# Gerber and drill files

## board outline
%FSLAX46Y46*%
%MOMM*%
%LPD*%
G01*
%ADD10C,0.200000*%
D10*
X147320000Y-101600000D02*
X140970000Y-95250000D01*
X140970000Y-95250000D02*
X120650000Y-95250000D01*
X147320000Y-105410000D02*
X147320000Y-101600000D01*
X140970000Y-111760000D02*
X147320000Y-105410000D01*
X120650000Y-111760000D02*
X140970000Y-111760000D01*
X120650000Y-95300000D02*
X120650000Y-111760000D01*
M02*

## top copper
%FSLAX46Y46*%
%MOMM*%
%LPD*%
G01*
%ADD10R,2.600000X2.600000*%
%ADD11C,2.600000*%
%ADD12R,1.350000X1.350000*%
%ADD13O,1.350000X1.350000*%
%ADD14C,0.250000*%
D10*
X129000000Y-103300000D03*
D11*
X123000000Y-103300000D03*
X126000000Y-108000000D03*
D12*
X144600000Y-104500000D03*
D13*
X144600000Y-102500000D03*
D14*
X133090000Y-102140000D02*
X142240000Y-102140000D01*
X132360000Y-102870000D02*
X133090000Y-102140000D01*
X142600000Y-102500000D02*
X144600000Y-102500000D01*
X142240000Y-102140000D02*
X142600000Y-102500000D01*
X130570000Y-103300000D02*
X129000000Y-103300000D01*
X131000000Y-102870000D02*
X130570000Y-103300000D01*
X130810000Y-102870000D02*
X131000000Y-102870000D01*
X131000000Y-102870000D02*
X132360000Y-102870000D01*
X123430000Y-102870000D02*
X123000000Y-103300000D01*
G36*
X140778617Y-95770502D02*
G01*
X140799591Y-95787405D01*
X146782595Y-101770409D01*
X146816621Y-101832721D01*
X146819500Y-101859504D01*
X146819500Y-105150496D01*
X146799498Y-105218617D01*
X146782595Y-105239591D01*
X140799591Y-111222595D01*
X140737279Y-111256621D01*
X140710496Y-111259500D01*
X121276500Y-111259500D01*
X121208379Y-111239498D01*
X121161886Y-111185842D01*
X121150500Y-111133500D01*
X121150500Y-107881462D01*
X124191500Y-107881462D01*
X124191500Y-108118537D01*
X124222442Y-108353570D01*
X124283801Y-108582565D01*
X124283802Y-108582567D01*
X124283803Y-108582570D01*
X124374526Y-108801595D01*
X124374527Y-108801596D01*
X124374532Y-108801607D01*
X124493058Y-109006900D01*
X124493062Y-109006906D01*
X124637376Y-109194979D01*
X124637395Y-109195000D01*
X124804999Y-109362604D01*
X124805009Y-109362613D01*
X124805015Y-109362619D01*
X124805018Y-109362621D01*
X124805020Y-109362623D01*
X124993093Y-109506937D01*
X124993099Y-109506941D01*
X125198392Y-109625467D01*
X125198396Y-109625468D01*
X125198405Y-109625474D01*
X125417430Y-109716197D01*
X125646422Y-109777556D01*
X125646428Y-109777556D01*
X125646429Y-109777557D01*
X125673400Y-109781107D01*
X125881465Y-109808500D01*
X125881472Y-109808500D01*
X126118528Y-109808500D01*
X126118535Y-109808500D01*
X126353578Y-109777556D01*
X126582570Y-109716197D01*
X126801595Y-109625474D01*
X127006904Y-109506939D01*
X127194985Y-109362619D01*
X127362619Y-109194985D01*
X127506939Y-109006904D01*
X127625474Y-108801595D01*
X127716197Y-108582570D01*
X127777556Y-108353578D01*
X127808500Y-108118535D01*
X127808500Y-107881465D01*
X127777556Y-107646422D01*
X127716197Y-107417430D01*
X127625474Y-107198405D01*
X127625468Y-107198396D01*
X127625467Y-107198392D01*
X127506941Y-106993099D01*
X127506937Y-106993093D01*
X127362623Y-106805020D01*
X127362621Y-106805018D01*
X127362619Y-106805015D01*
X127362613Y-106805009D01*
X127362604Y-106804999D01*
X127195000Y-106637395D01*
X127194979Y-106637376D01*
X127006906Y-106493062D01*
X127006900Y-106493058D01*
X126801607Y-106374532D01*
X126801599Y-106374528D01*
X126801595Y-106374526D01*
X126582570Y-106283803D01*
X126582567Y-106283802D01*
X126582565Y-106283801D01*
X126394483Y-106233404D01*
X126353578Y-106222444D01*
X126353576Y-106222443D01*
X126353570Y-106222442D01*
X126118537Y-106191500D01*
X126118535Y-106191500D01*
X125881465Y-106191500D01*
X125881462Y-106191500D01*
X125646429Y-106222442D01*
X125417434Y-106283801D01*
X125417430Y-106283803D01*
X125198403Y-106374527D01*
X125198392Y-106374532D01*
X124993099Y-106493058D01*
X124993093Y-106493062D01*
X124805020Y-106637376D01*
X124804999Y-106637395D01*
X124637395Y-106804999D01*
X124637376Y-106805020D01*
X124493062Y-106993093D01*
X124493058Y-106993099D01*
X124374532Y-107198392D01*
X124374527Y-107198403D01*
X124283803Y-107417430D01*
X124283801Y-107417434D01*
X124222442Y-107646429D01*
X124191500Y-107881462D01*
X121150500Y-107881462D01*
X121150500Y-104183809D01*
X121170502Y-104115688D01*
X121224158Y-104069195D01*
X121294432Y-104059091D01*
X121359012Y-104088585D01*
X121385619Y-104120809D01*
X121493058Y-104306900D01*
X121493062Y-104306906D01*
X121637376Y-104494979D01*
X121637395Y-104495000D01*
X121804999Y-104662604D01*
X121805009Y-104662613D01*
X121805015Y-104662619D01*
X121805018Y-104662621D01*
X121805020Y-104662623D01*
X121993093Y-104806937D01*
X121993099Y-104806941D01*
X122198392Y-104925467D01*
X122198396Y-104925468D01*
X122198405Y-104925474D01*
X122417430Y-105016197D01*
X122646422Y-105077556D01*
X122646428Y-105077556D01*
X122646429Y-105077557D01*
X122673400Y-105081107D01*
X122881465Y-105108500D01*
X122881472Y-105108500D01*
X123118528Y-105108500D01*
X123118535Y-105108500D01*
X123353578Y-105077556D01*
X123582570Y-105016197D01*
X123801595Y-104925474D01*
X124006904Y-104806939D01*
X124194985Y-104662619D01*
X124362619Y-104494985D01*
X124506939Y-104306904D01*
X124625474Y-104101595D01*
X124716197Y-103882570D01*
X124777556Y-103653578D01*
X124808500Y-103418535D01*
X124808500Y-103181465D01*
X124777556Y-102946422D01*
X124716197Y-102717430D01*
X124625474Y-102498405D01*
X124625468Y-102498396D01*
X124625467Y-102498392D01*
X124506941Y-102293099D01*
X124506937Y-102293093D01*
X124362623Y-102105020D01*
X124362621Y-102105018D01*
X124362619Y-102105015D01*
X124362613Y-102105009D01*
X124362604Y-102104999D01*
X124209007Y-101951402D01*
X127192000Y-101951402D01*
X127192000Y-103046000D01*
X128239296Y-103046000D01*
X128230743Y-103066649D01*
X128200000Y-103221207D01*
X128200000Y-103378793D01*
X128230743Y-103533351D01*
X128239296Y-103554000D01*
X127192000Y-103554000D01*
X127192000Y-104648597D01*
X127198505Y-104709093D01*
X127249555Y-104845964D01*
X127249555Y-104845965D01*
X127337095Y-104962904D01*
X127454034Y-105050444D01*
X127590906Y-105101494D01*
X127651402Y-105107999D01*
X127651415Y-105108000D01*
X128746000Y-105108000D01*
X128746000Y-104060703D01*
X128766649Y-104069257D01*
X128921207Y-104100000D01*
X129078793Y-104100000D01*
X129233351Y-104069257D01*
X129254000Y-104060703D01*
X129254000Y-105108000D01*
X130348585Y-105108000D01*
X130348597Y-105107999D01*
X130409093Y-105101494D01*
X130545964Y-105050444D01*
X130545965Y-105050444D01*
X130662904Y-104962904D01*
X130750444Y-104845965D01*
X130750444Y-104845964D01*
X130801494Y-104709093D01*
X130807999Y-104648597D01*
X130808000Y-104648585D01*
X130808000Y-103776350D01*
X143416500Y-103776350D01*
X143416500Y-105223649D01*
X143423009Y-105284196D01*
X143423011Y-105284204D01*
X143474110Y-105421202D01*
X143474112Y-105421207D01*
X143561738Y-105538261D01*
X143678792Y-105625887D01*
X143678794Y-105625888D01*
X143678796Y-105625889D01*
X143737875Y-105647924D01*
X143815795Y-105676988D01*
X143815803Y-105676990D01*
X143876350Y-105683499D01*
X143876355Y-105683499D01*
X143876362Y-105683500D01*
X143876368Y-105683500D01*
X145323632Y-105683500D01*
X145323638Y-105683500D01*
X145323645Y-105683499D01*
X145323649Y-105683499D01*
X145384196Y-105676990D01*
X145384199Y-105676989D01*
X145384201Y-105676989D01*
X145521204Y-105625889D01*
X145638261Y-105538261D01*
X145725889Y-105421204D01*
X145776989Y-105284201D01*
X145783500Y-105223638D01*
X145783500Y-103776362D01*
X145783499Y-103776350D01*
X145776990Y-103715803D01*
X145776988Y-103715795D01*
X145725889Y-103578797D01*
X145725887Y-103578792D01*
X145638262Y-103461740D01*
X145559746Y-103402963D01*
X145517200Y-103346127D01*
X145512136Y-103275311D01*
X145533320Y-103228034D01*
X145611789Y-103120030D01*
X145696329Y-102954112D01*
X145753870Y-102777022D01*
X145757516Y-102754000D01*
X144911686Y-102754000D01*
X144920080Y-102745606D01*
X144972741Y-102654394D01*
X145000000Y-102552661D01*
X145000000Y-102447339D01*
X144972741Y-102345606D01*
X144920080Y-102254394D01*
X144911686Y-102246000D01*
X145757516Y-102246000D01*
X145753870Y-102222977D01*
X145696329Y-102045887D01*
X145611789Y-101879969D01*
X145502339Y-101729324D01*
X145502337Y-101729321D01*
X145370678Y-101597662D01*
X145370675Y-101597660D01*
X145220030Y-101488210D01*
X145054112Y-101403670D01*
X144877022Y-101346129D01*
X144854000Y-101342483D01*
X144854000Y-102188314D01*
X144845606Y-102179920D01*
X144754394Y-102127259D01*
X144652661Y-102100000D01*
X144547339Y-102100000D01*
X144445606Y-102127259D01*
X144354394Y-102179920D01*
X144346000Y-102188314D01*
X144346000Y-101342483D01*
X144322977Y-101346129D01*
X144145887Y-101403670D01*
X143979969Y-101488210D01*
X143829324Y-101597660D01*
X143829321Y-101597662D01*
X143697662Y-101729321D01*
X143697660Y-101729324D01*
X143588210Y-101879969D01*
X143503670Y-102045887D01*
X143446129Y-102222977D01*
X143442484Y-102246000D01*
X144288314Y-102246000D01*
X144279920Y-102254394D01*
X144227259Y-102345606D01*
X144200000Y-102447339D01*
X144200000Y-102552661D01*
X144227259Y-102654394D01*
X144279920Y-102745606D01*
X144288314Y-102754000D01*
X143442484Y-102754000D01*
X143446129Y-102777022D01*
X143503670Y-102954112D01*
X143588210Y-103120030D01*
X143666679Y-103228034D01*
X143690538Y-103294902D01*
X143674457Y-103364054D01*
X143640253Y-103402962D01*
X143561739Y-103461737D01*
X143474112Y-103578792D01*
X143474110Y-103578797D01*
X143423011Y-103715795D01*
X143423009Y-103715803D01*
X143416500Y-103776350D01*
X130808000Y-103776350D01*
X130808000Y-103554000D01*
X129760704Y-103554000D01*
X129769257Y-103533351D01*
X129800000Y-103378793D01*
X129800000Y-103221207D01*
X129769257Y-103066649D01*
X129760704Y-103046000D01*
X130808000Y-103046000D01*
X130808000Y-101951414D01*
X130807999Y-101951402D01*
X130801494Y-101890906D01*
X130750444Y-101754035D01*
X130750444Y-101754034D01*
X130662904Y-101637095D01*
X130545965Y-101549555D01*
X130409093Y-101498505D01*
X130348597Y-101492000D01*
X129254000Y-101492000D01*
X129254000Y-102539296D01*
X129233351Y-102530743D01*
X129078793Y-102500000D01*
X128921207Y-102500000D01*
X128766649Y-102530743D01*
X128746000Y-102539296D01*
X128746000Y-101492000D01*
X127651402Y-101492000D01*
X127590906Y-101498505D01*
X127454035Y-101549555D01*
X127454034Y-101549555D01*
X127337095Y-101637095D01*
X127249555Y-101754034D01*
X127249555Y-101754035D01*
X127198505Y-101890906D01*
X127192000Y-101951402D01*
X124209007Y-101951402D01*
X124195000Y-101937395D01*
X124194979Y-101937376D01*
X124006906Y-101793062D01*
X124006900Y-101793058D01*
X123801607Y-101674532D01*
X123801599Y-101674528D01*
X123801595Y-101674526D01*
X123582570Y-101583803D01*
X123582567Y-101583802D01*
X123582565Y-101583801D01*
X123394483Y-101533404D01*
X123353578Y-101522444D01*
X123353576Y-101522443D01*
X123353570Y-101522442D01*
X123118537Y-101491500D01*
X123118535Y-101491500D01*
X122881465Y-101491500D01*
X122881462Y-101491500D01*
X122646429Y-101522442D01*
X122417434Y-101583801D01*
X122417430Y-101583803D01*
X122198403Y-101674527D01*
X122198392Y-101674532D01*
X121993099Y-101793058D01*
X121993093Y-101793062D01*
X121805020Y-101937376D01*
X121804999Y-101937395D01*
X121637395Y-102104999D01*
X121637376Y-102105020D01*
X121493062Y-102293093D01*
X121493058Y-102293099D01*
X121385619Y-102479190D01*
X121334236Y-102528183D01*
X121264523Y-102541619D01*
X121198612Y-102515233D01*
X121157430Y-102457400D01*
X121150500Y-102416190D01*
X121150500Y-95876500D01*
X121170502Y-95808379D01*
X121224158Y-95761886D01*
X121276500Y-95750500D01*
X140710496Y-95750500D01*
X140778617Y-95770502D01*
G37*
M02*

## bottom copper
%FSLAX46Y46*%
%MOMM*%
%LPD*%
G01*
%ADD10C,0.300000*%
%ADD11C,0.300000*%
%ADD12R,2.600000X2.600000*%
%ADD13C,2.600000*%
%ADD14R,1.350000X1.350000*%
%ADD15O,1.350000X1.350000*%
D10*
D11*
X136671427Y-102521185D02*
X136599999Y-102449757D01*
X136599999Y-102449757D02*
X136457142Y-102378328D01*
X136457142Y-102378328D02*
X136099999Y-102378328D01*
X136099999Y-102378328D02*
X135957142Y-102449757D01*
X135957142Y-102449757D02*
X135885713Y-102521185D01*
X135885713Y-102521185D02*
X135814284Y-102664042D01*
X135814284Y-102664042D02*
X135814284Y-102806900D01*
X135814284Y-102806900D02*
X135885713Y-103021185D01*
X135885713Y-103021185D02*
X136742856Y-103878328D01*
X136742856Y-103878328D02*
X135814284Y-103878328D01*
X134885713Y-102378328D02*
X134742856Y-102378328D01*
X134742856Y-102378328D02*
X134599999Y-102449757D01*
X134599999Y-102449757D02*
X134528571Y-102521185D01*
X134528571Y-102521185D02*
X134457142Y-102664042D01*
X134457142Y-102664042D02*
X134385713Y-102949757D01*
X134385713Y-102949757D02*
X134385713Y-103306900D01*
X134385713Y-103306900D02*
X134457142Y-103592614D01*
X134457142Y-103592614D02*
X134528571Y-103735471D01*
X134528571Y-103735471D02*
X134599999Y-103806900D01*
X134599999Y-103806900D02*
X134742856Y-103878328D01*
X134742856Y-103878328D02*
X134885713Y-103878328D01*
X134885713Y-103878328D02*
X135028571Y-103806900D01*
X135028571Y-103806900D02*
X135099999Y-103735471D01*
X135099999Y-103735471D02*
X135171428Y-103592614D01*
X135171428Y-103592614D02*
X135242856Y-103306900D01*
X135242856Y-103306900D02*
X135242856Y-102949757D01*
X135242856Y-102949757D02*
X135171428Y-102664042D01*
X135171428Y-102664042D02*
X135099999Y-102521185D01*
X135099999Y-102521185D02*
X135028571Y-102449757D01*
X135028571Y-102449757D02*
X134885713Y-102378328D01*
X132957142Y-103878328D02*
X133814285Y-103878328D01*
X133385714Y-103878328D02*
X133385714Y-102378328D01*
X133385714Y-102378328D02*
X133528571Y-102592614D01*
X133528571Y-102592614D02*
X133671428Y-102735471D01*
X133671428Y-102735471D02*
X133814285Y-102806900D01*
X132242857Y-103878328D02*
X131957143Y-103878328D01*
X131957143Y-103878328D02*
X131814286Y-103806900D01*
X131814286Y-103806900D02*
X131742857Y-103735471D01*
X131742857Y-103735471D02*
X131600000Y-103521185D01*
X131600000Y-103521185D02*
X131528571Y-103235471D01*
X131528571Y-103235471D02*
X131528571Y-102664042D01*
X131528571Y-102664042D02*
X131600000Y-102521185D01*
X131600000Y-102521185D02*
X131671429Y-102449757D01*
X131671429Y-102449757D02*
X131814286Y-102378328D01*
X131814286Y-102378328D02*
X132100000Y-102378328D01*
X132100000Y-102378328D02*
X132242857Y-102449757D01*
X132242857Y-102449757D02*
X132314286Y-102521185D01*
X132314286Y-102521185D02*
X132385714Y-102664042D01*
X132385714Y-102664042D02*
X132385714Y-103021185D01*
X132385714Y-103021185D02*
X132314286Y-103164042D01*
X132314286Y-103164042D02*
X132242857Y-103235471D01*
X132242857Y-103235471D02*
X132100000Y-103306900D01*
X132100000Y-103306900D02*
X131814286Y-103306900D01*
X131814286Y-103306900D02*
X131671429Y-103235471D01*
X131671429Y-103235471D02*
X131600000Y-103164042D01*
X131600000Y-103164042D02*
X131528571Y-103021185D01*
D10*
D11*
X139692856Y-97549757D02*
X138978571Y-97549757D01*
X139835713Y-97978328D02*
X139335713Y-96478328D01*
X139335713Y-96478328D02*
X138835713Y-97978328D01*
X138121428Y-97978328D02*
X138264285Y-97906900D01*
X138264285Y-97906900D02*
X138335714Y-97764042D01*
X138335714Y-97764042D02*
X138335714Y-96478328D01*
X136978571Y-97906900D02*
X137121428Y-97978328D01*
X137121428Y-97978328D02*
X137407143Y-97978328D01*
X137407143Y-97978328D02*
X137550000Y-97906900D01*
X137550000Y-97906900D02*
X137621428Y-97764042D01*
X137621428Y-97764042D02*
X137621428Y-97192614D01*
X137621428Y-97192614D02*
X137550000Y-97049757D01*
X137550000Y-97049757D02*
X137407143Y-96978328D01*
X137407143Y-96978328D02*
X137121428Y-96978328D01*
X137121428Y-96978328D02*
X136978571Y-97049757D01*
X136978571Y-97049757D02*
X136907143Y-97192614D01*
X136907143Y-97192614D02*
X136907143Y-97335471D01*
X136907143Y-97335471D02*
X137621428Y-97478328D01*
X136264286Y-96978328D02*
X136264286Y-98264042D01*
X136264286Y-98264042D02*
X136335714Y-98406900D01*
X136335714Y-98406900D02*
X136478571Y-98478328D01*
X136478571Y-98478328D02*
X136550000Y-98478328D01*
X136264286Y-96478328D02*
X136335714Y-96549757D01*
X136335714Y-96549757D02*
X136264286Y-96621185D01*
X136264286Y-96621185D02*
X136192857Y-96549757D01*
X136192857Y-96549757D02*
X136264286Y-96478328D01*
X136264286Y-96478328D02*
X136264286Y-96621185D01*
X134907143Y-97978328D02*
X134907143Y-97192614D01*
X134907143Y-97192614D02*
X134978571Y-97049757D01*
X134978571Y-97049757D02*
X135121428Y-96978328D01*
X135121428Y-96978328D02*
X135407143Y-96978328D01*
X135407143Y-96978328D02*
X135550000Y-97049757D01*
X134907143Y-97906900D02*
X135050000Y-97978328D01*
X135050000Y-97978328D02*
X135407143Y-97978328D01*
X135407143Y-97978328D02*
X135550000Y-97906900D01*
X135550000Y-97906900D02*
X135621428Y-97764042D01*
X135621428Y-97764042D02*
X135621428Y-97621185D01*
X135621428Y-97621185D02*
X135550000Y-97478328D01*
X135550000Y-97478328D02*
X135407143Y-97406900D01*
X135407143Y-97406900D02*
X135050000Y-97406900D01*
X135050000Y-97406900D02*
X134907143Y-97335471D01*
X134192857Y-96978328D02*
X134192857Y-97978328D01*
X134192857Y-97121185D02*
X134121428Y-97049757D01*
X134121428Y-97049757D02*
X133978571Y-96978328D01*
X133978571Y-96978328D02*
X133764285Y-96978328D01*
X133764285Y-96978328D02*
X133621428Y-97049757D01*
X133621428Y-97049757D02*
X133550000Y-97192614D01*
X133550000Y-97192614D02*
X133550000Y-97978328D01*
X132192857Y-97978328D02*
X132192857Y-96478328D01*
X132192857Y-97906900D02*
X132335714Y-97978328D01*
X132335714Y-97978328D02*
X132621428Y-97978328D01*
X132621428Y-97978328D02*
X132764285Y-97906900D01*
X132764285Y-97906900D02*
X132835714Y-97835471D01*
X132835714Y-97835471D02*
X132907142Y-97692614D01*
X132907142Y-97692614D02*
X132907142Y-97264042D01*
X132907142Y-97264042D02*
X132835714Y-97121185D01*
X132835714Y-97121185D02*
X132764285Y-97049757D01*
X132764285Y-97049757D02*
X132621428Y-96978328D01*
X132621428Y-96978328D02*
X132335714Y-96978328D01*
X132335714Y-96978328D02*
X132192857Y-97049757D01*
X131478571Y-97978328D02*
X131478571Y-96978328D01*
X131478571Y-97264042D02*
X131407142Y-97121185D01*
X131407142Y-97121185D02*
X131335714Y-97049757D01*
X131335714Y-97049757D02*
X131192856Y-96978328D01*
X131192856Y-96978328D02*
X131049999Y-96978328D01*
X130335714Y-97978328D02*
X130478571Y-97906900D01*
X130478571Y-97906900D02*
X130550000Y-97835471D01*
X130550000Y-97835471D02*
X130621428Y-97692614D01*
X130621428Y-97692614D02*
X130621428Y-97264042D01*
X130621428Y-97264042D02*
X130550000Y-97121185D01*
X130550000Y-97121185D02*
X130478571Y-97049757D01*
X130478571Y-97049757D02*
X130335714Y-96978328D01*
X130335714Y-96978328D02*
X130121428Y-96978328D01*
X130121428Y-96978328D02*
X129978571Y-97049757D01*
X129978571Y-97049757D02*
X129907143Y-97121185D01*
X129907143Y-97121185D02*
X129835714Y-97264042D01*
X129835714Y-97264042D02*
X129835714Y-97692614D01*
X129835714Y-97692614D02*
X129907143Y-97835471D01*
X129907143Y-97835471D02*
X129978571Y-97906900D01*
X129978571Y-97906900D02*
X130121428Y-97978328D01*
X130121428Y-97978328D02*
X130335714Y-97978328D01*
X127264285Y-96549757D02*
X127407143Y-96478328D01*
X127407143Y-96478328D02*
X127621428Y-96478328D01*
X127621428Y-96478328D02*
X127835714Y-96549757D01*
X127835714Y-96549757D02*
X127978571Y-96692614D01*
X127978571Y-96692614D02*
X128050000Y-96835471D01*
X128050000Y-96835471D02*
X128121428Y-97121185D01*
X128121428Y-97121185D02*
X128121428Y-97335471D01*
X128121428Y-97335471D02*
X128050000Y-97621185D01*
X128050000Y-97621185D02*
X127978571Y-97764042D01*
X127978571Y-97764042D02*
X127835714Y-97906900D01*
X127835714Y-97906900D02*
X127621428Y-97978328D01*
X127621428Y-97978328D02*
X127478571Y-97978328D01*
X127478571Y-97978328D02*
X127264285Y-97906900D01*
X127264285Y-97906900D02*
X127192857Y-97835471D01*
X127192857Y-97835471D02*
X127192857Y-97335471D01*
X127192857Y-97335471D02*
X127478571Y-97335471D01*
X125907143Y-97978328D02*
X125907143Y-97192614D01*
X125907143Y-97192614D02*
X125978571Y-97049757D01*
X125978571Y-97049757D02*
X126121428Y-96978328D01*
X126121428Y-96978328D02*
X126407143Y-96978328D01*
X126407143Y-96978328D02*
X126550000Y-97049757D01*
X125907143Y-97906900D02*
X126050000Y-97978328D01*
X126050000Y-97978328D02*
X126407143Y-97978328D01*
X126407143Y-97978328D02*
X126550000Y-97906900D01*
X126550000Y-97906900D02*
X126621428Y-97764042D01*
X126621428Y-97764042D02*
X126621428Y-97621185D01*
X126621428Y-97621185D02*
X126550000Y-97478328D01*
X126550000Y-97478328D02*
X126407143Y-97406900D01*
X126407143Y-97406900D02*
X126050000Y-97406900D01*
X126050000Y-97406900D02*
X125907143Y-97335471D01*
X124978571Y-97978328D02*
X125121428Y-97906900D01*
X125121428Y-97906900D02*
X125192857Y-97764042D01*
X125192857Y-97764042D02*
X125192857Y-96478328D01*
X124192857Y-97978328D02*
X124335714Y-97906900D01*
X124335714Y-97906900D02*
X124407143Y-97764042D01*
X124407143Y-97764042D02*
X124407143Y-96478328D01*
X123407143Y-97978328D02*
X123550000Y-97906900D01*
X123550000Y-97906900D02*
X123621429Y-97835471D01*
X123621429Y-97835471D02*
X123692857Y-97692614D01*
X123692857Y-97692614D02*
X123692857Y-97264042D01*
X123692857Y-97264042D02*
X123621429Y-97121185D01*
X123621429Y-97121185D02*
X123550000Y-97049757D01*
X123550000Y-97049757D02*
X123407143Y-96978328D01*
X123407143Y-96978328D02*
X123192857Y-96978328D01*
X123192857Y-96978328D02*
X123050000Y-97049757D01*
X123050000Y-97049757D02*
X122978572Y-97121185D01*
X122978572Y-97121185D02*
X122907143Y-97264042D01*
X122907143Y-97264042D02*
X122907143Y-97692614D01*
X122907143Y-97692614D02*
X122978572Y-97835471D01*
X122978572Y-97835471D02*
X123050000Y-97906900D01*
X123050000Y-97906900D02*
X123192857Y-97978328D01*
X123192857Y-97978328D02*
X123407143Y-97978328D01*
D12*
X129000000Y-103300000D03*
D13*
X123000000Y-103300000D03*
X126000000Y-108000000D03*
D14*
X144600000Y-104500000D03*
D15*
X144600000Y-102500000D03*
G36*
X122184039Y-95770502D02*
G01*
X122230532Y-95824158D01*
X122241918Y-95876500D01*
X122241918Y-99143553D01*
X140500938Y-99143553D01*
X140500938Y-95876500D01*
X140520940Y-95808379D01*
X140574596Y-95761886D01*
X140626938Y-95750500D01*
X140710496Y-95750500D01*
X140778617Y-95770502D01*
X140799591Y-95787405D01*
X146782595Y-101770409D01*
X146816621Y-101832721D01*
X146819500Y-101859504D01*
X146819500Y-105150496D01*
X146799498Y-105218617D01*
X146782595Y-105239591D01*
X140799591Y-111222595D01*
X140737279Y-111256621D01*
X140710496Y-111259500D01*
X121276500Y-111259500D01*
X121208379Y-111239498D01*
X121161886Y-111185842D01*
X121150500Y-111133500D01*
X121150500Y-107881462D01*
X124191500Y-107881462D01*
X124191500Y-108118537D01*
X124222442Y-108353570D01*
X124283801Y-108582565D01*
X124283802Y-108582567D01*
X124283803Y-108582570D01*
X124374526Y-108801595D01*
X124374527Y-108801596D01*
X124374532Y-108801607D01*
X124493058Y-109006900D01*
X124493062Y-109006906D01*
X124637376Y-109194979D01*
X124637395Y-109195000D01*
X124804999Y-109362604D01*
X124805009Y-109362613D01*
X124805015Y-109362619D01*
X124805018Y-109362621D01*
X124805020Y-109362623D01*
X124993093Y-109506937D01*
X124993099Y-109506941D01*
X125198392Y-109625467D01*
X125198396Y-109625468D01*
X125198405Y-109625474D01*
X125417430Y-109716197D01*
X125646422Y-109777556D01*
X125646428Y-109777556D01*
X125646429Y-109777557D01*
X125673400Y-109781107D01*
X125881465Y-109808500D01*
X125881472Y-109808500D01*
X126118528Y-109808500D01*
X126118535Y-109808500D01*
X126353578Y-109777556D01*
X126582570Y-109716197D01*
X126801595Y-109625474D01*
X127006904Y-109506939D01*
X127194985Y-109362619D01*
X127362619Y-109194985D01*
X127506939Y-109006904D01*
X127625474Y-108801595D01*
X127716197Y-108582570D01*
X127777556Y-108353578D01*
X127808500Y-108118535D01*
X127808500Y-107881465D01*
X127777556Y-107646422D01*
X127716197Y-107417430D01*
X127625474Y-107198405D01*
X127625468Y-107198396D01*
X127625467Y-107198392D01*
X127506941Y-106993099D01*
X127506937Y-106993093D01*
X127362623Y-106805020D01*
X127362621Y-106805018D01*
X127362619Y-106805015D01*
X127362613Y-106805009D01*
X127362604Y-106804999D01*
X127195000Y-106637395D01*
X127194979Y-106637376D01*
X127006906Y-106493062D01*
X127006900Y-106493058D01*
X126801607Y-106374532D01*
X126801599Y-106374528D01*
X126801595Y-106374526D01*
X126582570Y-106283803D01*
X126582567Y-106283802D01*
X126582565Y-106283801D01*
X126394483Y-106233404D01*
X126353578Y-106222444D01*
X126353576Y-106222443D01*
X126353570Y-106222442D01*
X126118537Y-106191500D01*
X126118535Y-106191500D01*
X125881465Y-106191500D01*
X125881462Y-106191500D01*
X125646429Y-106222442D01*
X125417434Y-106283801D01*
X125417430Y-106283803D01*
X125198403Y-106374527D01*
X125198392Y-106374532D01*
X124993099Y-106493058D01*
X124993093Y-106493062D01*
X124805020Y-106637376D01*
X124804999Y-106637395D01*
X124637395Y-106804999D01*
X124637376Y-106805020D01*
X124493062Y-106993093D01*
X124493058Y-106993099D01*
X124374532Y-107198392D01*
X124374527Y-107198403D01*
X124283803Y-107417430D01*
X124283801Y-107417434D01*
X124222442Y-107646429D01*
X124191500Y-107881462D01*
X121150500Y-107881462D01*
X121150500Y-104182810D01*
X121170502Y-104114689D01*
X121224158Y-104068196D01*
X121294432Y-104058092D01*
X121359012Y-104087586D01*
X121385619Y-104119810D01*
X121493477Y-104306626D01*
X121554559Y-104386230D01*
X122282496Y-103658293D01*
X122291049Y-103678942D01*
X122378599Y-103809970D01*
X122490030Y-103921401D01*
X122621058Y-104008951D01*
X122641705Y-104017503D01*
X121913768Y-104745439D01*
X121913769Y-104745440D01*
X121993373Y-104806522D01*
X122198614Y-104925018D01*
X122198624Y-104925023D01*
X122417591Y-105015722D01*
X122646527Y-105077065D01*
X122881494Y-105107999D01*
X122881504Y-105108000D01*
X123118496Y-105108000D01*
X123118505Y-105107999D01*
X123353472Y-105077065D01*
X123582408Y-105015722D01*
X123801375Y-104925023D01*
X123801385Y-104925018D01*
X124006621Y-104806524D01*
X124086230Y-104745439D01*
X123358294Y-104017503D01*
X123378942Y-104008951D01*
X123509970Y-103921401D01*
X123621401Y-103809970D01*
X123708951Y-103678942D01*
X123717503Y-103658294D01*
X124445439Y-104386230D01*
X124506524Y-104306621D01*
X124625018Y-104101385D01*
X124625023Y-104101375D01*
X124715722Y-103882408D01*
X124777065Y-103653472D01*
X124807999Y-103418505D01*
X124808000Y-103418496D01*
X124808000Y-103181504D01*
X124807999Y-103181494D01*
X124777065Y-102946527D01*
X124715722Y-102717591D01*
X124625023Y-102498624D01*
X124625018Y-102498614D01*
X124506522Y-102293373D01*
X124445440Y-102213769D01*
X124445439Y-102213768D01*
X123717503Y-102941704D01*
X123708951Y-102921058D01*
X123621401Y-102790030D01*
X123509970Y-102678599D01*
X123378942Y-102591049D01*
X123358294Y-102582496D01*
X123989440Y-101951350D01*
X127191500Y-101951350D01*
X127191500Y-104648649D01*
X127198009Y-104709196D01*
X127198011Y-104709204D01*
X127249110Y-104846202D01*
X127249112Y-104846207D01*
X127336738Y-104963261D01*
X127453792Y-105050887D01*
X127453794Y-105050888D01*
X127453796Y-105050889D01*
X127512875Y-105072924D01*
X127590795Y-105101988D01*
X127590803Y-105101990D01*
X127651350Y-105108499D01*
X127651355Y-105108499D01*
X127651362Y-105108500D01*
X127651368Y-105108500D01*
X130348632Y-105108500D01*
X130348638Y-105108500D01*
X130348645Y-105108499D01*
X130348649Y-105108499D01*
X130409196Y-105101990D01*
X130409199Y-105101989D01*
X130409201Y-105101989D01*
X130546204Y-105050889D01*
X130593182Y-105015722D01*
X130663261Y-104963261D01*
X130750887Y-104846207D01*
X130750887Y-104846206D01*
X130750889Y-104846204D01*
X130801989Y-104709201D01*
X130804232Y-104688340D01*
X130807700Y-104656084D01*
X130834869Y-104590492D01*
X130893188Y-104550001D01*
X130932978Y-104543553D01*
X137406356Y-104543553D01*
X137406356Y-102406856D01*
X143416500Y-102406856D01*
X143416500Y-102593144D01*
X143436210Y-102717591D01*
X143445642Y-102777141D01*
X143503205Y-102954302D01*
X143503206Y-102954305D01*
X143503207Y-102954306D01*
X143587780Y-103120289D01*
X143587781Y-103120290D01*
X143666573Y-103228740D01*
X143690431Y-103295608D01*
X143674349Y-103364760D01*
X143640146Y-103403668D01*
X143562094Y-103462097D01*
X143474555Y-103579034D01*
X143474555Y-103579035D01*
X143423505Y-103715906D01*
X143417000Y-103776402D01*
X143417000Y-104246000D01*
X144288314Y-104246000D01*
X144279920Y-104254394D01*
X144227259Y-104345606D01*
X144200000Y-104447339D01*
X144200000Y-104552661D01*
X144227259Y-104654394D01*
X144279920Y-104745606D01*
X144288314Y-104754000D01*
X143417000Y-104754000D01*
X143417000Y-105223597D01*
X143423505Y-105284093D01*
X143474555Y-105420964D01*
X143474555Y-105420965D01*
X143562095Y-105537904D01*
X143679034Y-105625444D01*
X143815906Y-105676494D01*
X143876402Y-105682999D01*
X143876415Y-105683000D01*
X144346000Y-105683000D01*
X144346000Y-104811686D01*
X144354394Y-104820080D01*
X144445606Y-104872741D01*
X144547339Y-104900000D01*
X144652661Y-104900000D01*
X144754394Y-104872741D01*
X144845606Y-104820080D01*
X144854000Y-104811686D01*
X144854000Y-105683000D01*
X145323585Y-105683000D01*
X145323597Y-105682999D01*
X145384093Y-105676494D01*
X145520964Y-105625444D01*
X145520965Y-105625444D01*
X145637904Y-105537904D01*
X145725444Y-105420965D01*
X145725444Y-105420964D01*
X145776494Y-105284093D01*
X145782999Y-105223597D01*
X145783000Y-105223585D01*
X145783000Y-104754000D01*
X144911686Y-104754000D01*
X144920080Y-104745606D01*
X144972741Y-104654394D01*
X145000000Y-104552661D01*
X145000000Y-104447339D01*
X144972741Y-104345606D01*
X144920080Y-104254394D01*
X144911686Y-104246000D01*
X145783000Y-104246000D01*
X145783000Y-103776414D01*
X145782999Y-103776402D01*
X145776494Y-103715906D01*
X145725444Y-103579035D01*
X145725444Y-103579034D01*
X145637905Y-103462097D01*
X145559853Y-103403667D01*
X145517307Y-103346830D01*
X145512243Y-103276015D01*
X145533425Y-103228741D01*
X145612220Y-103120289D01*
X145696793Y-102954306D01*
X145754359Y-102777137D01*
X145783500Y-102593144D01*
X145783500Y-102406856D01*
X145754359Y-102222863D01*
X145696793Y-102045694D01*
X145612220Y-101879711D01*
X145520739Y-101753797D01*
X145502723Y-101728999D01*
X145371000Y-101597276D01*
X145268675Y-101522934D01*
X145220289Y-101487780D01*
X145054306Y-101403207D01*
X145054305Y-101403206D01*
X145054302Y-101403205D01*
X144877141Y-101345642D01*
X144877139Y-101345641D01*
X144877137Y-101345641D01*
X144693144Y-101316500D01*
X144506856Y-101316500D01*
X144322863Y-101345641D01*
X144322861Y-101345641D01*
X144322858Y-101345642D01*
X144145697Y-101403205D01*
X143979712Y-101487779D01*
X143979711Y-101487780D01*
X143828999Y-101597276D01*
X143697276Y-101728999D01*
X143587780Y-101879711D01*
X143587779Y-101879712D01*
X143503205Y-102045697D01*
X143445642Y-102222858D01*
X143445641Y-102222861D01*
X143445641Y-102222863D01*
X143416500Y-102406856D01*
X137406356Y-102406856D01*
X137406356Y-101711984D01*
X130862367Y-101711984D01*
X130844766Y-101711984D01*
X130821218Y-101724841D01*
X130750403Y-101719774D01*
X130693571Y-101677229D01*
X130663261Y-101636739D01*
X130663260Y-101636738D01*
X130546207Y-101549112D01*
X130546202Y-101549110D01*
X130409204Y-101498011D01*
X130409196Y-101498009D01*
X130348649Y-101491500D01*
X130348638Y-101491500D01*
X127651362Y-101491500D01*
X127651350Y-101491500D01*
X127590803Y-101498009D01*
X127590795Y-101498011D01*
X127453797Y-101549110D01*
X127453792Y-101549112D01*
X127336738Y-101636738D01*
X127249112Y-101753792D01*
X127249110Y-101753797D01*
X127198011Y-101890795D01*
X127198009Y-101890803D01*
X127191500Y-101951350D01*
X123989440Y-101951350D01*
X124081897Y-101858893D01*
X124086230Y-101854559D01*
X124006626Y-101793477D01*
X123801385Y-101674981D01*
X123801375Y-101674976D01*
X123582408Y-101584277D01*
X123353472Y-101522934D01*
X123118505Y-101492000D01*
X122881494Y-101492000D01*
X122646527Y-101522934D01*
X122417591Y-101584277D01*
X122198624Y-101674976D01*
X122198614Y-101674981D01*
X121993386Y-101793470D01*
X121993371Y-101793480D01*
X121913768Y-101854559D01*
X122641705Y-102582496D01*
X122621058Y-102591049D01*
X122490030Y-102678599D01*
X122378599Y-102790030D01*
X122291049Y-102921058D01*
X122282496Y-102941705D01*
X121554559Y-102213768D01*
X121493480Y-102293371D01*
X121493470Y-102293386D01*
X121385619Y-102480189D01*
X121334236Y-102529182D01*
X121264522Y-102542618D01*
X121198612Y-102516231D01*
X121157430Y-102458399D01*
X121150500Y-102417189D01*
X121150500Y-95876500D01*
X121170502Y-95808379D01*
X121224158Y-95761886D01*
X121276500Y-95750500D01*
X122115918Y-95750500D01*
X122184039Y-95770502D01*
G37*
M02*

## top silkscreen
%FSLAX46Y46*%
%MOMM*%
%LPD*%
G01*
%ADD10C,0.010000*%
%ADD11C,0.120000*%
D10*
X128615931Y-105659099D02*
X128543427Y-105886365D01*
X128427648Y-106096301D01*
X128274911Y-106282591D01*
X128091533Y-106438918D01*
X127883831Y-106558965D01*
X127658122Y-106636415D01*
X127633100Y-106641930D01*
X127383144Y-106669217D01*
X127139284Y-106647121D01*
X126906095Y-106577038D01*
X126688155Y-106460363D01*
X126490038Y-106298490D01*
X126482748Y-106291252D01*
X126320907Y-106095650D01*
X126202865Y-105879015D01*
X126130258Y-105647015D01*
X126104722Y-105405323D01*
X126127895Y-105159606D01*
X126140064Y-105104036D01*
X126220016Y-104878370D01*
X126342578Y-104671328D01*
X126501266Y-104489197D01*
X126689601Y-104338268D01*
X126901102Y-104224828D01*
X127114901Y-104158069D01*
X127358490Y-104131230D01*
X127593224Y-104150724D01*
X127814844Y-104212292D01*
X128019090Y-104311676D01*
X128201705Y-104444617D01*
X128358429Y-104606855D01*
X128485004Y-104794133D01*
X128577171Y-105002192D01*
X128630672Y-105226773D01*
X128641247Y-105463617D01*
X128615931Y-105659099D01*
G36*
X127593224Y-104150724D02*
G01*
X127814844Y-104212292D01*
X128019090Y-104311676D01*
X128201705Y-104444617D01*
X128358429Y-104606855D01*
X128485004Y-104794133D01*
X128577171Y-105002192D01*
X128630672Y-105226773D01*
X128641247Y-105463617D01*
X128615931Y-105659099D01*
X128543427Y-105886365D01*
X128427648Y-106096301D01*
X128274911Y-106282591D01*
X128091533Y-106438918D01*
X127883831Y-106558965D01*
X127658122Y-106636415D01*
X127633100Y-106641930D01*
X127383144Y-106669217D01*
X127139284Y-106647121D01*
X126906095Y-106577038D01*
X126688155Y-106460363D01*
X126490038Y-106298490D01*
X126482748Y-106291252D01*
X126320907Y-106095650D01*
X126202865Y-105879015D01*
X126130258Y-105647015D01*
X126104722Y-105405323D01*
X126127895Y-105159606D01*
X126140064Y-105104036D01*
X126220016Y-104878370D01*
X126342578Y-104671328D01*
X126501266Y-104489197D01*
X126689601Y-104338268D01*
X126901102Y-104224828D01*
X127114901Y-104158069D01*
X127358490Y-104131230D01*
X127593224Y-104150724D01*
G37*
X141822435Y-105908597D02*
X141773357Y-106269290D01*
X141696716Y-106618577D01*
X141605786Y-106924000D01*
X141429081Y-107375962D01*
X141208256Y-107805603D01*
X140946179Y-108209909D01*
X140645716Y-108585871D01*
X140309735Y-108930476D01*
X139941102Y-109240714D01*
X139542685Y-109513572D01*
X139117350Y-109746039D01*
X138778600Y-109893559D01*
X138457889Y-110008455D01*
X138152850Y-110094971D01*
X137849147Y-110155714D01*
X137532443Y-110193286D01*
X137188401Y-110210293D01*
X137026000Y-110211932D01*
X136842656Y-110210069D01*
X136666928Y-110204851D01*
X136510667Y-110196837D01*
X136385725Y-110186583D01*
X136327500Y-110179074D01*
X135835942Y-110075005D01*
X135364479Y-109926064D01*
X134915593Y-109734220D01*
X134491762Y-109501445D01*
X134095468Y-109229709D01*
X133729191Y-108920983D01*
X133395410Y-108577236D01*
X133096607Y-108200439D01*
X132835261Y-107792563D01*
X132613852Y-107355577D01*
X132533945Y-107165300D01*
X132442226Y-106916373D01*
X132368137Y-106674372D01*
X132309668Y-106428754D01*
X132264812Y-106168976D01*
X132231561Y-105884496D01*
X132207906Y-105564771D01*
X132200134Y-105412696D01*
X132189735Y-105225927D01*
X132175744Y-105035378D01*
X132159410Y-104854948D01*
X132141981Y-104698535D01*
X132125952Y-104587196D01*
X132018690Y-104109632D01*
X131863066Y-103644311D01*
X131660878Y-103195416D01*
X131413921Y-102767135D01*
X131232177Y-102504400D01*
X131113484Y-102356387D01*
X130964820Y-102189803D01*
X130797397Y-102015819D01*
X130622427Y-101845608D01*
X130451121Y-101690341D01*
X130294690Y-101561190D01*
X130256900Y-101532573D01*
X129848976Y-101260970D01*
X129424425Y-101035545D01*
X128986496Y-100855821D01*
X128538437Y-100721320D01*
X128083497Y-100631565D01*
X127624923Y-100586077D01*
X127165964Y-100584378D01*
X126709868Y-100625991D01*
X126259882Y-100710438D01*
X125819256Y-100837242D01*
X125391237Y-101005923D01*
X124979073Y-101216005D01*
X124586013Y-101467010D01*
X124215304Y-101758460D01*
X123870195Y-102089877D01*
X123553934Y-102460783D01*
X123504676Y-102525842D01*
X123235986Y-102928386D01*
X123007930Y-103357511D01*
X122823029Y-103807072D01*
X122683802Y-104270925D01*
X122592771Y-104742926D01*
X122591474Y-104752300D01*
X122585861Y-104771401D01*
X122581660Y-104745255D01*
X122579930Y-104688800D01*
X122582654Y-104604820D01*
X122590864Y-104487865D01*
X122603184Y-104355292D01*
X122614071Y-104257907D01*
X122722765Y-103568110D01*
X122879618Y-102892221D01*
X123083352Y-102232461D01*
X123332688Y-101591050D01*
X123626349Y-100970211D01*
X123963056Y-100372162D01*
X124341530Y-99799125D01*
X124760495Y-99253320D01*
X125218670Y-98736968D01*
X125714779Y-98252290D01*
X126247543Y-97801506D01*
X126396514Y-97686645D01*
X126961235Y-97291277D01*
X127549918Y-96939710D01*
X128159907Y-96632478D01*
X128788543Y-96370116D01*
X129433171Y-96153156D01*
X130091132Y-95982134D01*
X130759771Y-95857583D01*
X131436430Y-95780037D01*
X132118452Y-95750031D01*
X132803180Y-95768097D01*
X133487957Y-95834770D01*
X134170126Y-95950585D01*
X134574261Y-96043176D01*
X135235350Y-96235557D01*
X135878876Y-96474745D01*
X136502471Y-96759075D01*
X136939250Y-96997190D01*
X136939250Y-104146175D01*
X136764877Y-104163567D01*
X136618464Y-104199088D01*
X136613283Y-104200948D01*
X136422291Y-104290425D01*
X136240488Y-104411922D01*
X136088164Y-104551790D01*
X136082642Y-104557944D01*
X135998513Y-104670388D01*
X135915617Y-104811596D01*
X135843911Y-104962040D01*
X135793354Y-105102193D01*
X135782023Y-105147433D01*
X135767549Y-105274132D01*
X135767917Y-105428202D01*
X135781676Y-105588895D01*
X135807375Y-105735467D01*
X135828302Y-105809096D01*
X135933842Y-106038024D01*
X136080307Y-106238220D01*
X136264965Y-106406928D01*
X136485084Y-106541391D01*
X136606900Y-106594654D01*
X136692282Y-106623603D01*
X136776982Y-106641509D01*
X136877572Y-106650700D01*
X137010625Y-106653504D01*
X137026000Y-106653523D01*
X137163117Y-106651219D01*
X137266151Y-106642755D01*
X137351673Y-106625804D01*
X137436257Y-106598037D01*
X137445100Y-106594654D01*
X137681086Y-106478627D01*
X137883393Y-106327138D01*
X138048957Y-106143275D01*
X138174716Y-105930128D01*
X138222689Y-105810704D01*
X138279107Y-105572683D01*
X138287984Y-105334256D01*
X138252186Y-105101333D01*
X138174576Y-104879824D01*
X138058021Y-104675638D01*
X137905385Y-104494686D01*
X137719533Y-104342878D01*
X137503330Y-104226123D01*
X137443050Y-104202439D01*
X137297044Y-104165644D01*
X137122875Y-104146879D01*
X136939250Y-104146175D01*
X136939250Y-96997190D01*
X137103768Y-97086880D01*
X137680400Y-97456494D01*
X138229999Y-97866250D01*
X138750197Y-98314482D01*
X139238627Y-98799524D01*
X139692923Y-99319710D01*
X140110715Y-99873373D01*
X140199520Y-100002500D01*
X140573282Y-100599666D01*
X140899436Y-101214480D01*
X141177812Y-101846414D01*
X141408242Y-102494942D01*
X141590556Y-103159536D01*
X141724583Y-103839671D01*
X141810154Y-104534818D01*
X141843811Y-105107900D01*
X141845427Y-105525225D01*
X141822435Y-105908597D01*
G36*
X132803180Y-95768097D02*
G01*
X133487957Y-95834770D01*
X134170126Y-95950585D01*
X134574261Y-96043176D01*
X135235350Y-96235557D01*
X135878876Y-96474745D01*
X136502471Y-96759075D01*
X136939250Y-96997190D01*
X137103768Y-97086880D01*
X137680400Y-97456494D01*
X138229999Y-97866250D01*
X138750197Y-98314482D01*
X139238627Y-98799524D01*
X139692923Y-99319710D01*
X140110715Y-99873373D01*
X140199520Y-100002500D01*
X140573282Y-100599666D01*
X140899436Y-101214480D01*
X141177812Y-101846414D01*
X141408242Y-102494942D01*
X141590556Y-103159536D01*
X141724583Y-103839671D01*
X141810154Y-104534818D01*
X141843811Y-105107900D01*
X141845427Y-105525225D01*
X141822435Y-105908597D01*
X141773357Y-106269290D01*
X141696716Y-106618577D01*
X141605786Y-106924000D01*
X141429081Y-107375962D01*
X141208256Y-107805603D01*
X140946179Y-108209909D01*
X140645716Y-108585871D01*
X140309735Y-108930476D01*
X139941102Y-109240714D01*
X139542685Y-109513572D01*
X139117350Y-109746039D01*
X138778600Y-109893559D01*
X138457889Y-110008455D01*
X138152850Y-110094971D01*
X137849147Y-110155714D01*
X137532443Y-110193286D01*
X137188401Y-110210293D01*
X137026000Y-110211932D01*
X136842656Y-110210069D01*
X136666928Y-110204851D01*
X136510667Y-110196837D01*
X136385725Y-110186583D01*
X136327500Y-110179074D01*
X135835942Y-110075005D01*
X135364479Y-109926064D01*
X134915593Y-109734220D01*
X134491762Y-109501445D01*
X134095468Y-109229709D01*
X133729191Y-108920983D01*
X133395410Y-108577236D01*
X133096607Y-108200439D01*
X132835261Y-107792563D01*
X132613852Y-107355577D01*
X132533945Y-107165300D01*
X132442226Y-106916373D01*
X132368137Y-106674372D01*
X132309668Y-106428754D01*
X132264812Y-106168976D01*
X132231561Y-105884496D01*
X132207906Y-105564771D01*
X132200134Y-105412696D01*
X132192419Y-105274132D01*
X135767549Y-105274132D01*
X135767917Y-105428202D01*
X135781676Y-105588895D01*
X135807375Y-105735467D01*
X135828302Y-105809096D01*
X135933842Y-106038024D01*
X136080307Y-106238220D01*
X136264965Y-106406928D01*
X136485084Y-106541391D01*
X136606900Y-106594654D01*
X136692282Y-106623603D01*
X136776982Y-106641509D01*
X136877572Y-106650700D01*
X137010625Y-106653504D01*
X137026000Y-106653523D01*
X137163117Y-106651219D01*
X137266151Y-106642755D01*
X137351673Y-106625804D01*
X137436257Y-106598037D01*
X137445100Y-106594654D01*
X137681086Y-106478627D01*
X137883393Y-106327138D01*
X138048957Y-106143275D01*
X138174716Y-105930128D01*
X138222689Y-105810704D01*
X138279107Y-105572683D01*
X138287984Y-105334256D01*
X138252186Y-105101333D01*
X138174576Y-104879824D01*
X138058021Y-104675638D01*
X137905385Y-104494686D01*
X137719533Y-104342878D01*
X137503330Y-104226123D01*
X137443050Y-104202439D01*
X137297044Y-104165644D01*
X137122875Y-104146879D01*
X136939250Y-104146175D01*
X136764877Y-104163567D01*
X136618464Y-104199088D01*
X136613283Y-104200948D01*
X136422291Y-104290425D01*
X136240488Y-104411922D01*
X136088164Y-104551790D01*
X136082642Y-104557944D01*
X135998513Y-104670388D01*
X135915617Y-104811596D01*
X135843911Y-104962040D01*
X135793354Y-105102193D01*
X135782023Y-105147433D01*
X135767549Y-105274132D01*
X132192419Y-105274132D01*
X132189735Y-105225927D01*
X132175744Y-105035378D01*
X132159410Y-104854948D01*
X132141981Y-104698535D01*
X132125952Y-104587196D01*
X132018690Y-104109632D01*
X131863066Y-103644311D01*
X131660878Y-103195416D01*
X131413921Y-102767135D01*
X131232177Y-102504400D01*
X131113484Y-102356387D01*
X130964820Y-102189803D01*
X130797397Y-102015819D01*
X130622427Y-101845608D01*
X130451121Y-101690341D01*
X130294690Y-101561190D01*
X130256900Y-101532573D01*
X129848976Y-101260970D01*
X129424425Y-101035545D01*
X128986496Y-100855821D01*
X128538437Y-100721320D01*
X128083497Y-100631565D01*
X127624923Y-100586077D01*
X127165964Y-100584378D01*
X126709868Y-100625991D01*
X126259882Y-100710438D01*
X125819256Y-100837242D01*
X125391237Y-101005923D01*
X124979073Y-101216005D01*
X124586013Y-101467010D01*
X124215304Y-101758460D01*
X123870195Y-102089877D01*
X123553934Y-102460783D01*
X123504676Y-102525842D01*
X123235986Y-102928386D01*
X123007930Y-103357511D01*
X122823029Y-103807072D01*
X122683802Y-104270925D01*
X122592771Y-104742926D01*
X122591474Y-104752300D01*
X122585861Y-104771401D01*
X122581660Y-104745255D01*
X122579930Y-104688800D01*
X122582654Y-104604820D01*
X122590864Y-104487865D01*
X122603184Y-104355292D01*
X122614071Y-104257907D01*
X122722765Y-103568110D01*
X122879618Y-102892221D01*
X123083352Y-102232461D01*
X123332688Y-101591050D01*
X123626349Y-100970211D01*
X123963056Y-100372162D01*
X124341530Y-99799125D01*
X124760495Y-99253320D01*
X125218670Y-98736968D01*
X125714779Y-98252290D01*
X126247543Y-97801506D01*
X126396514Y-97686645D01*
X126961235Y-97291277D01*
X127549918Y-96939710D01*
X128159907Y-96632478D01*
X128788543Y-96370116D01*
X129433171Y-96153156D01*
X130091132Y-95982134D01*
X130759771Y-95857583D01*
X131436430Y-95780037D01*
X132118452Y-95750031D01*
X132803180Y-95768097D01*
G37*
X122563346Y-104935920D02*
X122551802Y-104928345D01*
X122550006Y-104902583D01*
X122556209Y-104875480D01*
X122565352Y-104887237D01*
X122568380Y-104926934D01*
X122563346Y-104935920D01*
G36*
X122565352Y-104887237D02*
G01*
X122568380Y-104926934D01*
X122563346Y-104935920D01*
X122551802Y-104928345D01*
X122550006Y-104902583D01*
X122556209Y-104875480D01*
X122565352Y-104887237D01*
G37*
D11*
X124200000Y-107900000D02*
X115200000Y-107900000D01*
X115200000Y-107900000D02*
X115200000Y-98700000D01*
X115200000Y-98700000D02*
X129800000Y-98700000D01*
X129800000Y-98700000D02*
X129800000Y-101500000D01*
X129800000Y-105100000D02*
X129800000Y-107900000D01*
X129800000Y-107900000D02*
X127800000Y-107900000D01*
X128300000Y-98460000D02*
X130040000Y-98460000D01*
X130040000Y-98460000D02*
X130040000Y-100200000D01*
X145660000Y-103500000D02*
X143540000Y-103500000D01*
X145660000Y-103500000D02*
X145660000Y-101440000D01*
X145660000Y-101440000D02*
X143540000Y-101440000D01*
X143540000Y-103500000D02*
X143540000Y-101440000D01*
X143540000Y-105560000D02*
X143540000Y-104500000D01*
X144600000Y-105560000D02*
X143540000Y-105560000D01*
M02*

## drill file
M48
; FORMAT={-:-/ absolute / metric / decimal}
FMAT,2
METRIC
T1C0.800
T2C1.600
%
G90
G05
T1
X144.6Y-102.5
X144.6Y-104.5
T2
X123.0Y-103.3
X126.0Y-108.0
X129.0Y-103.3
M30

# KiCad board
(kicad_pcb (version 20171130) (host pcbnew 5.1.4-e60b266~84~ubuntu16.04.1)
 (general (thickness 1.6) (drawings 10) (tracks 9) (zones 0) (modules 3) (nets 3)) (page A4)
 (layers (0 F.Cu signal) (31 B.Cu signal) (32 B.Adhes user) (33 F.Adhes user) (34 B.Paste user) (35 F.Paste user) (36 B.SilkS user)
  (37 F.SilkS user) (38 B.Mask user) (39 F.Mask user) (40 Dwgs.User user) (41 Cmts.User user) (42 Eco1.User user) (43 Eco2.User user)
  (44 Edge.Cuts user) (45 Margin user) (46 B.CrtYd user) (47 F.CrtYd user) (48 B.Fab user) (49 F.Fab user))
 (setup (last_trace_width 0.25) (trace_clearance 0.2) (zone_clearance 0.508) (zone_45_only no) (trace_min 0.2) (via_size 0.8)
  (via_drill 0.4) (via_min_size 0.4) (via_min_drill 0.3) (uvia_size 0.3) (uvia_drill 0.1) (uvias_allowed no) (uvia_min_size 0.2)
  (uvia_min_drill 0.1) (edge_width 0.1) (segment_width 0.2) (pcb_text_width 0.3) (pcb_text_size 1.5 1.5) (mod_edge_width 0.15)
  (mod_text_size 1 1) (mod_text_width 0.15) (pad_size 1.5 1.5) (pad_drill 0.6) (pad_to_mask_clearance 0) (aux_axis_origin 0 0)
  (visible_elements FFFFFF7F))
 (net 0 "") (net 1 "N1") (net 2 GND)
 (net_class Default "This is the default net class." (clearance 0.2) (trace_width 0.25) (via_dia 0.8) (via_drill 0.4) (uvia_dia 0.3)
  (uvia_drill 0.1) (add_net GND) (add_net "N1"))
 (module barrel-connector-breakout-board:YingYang (layer F.Cu) (at 132.2 105.4 270)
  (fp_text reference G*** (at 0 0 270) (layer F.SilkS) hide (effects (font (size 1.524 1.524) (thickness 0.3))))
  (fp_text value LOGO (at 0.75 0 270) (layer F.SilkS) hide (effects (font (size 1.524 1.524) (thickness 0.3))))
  (fp_poly
   (pts (xy 0.259099 3.584069) (xy 0.486365 3.656573) (xy 0.696301 3.772352) (xy 0.882591 3.925089) (xy 1.038918 4.108467)
    (xy 1.158965 4.316169) (xy 1.236415 4.541878) (xy 1.24193 4.5669) (xy 1.269217 4.816856) (xy 1.247121 5.060716) (xy 1.177038 5.293905)
    (xy 1.060363 5.511845) (xy 0.89849 5.709962) (xy 0.891252 5.717252) (xy 0.69565 5.879093) (xy 0.479015 5.997135) (xy 0.247015 6.069742)
    (xy 0.005323 6.095278) (xy -0.240394 6.072105) (xy -0.295964 6.059936) (xy -0.52163 5.979984) (xy -0.728672 5.857422)
    (xy -0.910803 5.698734) (xy -1.061732 5.510399) (xy -1.175172 5.298898) (xy -1.241931 5.085099) (xy -1.26877 4.84151)
    (xy -1.249276 4.606776) (xy -1.187708 4.385156) (xy -1.088324 4.18091) (xy -0.955383 3.998295) (xy -0.793145 3.841571)
    (xy -0.605867 3.714996) (xy -0.397808 3.622829) (xy -0.173227 3.569328) (xy 0.063617 3.558753) (xy 0.259099 3.584069))
   (layer F.SilkS) (width 0.01))
  (fp_poly
   (pts (xy 0.508597 -9.622435) (xy 0.86929 -9.573357) (xy 1.218577 -9.496716) (xy 1.524 -9.405786) (xy 1.975962 -9.229081)
    (xy 2.405603 -9.008256) (xy 2.809909 -8.746179) (xy 3.185871 -8.445716) (xy 3.530476 -8.109735) (xy 3.840714 -7.741102)
    (xy 4.113572 -7.342685) (xy 4.346039 -6.91735) (xy 4.493559 -6.5786) (xy 4.608455 -6.257889) (xy 4.694971 -5.95285)
    (xy 4.755714 -5.649147) (xy 4.793286 -5.332443) (xy 4.810293 -4.988401) (xy 4.811932 -4.826) (xy 4.810069 -4.642656)
    (xy 4.804851 -4.466928) (xy 4.796837 -4.310667) (xy 4.786583 -4.185725) (xy 4.779074 -4.1275) (xy 4.675005 -3.635942)
    (xy 4.526064 -3.164479) (xy 4.33422 -2.715593) (xy 4.101445 -2.291762) (xy 3.829709 -1.895468) (xy 3.520983 -1.529191)
    (xy 3.177236 -1.19541) (xy 2.800439 -0.896607) (xy 2.392563 -0.635261) (xy 1.955577 -0.413852) (xy 1.7653 -0.333945)
    (xy 1.516373 -0.242226) (xy 1.274372 -0.168137) (xy 1.028754 -0.109668) (xy 0.768976 -0.064812) (xy 0.484496 -0.031561)
    (xy 0.164771 -0.007906) (xy 0.012696 -0.000134) (xy -0.174073 0.010265) (xy -0.364622 0.024256) (xy -0.545052 0.04059)
    (xy -0.701465 0.058019) (xy -0.812804 0.074048) (xy -1.290368 0.18131) (xy -1.755689 0.336934) (xy -2.204584 0.539122)
    (xy -2.632865 0.786079) (xy -2.8956 0.967823) (xy -3.043613 1.086516) (xy -3.210197 1.23518) (xy -3.384181 1.402603)
    (xy -3.554392 1.577573) (xy -3.709659 1.748879) (xy -3.83881 1.90531) (xy -3.867427 1.9431) (xy -4.13903 2.351024)
    (xy -4.364455 2.775575) (xy -4.544179 3.213504) (xy -4.67868 3.661563) (xy -4.768435 4.116503) (xy -4.813923 4.575077)
    (xy -4.815622 5.034036) (xy -4.774009 5.490132) (xy -4.689562 5.940118) (xy -4.562758 6.380744) (xy -4.394077 6.808763)
    (xy -4.183995 7.220927) (xy -3.93299 7.613987) (xy -3.64154 7.984696) (xy -3.310123 8.329805) (xy -2.939217 8.646066)
    (xy -2.874158 8.695324) (xy -2.471614 8.964014) (xy -2.042489 9.19207) (xy -1.592928 9.376971) (xy -1.129075 9.516198)
    (xy -0.657074 9.607229) (xy -0.6477 9.608526) (xy -0.628599 9.614139) (xy -0.654745 9.61834) (xy -0.7112 9.62007) (xy -0.79518 9.617346)
    (xy -0.912135 9.609136) (xy -1.044708 9.596816) (xy -1.142093 9.585929) (xy -1.83189 9.477235) (xy -2.507779 9.320382)
    (xy -3.167539 9.116648) (xy -3.80895 8.867312) (xy -4.429789 8.573651) (xy -5.027838 8.236944) (xy -5.600875 7.85847)
    (xy -6.14668 7.439505) (xy -6.663032 6.98133) (xy -7.14771 6.485221) (xy -7.598494 5.952457) (xy -7.713355 5.803486)
    (xy -8.108723 5.238765) (xy -8.46029 4.650082) (xy -8.767522 4.040093) (xy -9.029884 3.411457) (xy -9.246844 2.766829)
    (xy -9.417866 2.108868) (xy -9.542417 1.440229) (xy -9.619963 0.76357) (xy -9.649969 0.081548) (xy -9.631903 -0.60318)
    (xy -9.56523 -1.287957) (xy -9.449415 -1.970126) (xy -9.356824 -2.374261) (xy -9.164443 -3.03535) (xy -8.925255 -3.678876)
    (xy -8.640925 -4.302471) (xy -8.40281 -4.73925) (xy -1.253825 -4.73925) (xy -1.236433 -4.564877) (xy -1.200912 -4.418464)
    (xy -1.199052 -4.413283) (xy -1.109575 -4.222291) (xy -0.988078 -4.040488) (xy -0.84821 -3.888164) (xy -0.842056 -3.882642)
    (xy -0.729612 -3.798513) (xy -0.588404 -3.715617) (xy -0.43796 -3.643911) (xy -0.297807 -3.593354) (xy -0.252567 -3.582023)
    (xy -0.125868 -3.567549) (xy 0.028202 -3.567917) (xy 0.188895 -3.581676) (xy 0.335467 -3.607375) (xy 0.409096 -3.628302)
    (xy 0.638024 -3.733842) (xy 0.83822 -3.880307) (xy 1.006928 -4.064965) (xy 1.141391 -4.285084) (xy 1.194654 -4.4069)
    (xy 1.223603 -4.492282) (xy 1.241509 -4.576982) (xy 1.2507 -4.677572) (xy 1.253504 -4.810625) (xy 1.253523 -4.826)
    (xy 1.251219 -4.963117) (xy 1.242755 -5.066151) (xy 1.225804 -5.151673) (xy 1.198037 -5.236257) (xy 1.194654 -5.2451)
    (xy 1.078627 -5.481086) (xy 0.927138 -5.683393) (xy 0.743275 -5.848957) (xy 0.530128 -5.974716) (xy 0.410704 -6.022689)
    (xy 0.172683 -6.079107) (xy -0.065744 -6.087984) (xy -0.298667 -6.052186) (xy -0.520176 -5.974576) (xy -0.724362 -5.858021)
    (xy -0.905314 -5.705385) (xy -1.057122 -5.519533) (xy -1.173877 -5.30333) (xy -1.197561 -5.24305) (xy -1.234356 -5.097044)
    (xy -1.253121 -4.922875) (xy -1.253825 -4.73925) (xy -8.40281 -4.73925) (xy -8.31312 -4.903768) (xy -7.943506 -5.4804)
    (xy -7.53375 -6.029999) (xy -7.085518 -6.550197) (xy -6.600476 -7.038627) (xy -6.08029 -7.492923) (xy -5.526627 -7.910715)
    (xy -5.3975 -7.99952) (xy -4.800334 -8.373282) (xy -4.18552 -8.699436) (xy -3.553586 -8.977812) (xy -2.905058 -9.208242)
    (xy -2.240464 -9.390556) (xy -1.560329 -9.524583) (xy -0.865182 -9.610154) (xy -0.2921 -9.643811) (xy 0.125225 -9.645427)
    (xy 0.508597 -9.622435))
   (layer F.SilkS) (width 0.01))
  (fp_poly
   (pts (xy -0.46408 9.636654) (xy -0.471655 9.648198) (xy -0.497417 9.649994) (xy -0.52452 9.643791) (xy -0.512763 9.634648)
    (xy -0.473066 9.63162) (xy -0.46408 9.636654))
   (layer F.SilkS) (width 0.01)))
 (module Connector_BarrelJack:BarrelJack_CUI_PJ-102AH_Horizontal (layer F.Cu) (at 129 103.3 270)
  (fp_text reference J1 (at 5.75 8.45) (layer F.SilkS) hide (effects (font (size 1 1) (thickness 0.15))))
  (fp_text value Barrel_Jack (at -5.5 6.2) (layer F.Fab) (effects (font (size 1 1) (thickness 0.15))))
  (fp_line (start 4.6 4.8) (end 4.6 13.8) (layer F.SilkS) (width 0.12))
  (fp_line (start 4.6 13.8) (end -4.6 13.8) (layer F.SilkS) (width 0.12))
  (fp_line (start -4.6 13.8) (end -4.6 -0.8) (layer F.SilkS) (width 0.12))
  (fp_line (start -4.6 -0.8) (end -1.8 -0.8) (layer F.SilkS) (width 0.12))
  (fp_line (start 1.8 -0.8) (end 4.6 -0.8) (layer F.SilkS) (width 0.12))
  (fp_line (start 4.6 -0.8) (end 4.6 1.2) (layer F.SilkS) (width 0.12))
  (fp_line (start -4.84 0.7) (end -4.84 -1.04) (layer F.SilkS) (width 0.12))
  (fp_line (start -4.84 -1.04) (end -3.1 -1.04) (layer F.SilkS) (width 0.12))
  (pad 1 thru_hole rect (at 0 0 270) (size 2.6 2.6) (drill 1.6) (layers *.Cu *.Mask) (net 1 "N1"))
  (pad 2 thru_hole circle (at 0 6 270) (size 2.6 2.6) (drill 1.6) (layers *.Cu *.Mask) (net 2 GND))
  (pad 3 thru_hole circle (at 4.7 3 270) (size 2.6 2.6) (drill 1.6) (layers *.Cu *.Mask)))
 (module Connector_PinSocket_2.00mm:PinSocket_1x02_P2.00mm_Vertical (layer F.Cu) (at 144.6 104.5 180)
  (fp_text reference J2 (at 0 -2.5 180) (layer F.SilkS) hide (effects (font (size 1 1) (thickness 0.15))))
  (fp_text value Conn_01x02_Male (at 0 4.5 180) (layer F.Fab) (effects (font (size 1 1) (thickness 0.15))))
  (fp_line (start -1.06 1) (end 1.06 1) (layer F.SilkS) (width 0.12))
  (fp_line (start -1.06 1) (end -1.06 3.06) (layer F.SilkS) (width 0.12))
  (fp_line (start -1.06 3.06) (end 1.06 3.06) (layer F.SilkS) (width 0.12))
  (fp_line (start 1.06 1) (end 1.06 3.06) (layer F.SilkS) (width 0.12))
  (fp_line (start 1.06 -1.06) (end 1.06 0) (layer F.SilkS) (width 0.12))
  (fp_line (start 0 -1.06) (end 1.06 -1.06) (layer F.SilkS) (width 0.12))
  (pad 1 thru_hole rect (at 0 0 180) (size 1.35 1.35) (drill 0.8) (layers *.Cu *.Mask) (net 2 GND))
  (pad 2 thru_hole oval (at 0 2 180) (size 1.35 1.35) (drill 0.8) (layers *.Cu *.Mask) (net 1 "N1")))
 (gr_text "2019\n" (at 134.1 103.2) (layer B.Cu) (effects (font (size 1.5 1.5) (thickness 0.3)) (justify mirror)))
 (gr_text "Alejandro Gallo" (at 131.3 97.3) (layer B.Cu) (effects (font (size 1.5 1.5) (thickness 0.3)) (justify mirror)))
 (gr_line (start 147.32 101.6) (end 140.97 95.25) (layer Edge.Cuts) (width 0.2))
 (gr_line (start 140.97 95.25) (end 120.65 95.25) (layer Edge.Cuts) (width 0.2))
 (gr_line (start 147.32 105.41) (end 147.32 101.6) (layer Edge.Cuts) (width 0.2))
 (gr_line (start 140.97 111.76) (end 147.32 105.41) (layer Edge.Cuts) (width 0.2))
 (gr_line (start 120.65 111.76) (end 140.97 111.76) (layer Edge.Cuts) (width 0.2))
 (gr_line (start 120.65 95.3) (end 120.65 111.76) (layer Edge.Cuts) (width 0.2))
 (segment (start 133.09 102.14) (end 142.24 102.14) (width 0.25) (layer F.Cu) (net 1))
 (segment (start 132.36 102.87) (end 133.09 102.14) (width 0.25) (layer F.Cu) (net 1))
 (segment (start 142.6 102.5) (end 144.6 102.5) (width 0.25) (layer F.Cu) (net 1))
 (segment (start 142.24 102.14) (end 142.6 102.5) (width 0.25) (layer F.Cu) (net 1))
 (segment (start 130.57 103.3) (end 129 103.3) (width 0.25) (layer F.Cu) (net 1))
 (segment (start 131 102.87) (end 130.57 103.3) (width 0.25) (layer F.Cu) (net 1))
 (segment (start 130.81 102.87) (end 131 102.87) (width 0.25) (layer F.Cu) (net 1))
 (segment (start 131 102.87) (end 132.36 102.87) (width 0.25) (layer F.Cu) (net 1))
 (segment (start 123.43 102.87) (end 123 103.3) (width 0.25) (layer F.Cu) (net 2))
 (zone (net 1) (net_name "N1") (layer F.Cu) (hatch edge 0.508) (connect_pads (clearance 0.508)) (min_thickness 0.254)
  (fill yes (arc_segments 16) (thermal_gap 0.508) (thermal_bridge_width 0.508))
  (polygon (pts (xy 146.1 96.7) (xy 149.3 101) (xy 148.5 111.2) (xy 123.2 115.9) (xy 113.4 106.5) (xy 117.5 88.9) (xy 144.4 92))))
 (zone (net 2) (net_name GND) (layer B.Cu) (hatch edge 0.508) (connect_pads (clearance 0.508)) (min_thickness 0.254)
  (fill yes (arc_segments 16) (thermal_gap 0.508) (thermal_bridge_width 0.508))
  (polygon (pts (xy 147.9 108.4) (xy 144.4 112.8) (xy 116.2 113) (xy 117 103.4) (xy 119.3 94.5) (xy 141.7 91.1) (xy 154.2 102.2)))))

